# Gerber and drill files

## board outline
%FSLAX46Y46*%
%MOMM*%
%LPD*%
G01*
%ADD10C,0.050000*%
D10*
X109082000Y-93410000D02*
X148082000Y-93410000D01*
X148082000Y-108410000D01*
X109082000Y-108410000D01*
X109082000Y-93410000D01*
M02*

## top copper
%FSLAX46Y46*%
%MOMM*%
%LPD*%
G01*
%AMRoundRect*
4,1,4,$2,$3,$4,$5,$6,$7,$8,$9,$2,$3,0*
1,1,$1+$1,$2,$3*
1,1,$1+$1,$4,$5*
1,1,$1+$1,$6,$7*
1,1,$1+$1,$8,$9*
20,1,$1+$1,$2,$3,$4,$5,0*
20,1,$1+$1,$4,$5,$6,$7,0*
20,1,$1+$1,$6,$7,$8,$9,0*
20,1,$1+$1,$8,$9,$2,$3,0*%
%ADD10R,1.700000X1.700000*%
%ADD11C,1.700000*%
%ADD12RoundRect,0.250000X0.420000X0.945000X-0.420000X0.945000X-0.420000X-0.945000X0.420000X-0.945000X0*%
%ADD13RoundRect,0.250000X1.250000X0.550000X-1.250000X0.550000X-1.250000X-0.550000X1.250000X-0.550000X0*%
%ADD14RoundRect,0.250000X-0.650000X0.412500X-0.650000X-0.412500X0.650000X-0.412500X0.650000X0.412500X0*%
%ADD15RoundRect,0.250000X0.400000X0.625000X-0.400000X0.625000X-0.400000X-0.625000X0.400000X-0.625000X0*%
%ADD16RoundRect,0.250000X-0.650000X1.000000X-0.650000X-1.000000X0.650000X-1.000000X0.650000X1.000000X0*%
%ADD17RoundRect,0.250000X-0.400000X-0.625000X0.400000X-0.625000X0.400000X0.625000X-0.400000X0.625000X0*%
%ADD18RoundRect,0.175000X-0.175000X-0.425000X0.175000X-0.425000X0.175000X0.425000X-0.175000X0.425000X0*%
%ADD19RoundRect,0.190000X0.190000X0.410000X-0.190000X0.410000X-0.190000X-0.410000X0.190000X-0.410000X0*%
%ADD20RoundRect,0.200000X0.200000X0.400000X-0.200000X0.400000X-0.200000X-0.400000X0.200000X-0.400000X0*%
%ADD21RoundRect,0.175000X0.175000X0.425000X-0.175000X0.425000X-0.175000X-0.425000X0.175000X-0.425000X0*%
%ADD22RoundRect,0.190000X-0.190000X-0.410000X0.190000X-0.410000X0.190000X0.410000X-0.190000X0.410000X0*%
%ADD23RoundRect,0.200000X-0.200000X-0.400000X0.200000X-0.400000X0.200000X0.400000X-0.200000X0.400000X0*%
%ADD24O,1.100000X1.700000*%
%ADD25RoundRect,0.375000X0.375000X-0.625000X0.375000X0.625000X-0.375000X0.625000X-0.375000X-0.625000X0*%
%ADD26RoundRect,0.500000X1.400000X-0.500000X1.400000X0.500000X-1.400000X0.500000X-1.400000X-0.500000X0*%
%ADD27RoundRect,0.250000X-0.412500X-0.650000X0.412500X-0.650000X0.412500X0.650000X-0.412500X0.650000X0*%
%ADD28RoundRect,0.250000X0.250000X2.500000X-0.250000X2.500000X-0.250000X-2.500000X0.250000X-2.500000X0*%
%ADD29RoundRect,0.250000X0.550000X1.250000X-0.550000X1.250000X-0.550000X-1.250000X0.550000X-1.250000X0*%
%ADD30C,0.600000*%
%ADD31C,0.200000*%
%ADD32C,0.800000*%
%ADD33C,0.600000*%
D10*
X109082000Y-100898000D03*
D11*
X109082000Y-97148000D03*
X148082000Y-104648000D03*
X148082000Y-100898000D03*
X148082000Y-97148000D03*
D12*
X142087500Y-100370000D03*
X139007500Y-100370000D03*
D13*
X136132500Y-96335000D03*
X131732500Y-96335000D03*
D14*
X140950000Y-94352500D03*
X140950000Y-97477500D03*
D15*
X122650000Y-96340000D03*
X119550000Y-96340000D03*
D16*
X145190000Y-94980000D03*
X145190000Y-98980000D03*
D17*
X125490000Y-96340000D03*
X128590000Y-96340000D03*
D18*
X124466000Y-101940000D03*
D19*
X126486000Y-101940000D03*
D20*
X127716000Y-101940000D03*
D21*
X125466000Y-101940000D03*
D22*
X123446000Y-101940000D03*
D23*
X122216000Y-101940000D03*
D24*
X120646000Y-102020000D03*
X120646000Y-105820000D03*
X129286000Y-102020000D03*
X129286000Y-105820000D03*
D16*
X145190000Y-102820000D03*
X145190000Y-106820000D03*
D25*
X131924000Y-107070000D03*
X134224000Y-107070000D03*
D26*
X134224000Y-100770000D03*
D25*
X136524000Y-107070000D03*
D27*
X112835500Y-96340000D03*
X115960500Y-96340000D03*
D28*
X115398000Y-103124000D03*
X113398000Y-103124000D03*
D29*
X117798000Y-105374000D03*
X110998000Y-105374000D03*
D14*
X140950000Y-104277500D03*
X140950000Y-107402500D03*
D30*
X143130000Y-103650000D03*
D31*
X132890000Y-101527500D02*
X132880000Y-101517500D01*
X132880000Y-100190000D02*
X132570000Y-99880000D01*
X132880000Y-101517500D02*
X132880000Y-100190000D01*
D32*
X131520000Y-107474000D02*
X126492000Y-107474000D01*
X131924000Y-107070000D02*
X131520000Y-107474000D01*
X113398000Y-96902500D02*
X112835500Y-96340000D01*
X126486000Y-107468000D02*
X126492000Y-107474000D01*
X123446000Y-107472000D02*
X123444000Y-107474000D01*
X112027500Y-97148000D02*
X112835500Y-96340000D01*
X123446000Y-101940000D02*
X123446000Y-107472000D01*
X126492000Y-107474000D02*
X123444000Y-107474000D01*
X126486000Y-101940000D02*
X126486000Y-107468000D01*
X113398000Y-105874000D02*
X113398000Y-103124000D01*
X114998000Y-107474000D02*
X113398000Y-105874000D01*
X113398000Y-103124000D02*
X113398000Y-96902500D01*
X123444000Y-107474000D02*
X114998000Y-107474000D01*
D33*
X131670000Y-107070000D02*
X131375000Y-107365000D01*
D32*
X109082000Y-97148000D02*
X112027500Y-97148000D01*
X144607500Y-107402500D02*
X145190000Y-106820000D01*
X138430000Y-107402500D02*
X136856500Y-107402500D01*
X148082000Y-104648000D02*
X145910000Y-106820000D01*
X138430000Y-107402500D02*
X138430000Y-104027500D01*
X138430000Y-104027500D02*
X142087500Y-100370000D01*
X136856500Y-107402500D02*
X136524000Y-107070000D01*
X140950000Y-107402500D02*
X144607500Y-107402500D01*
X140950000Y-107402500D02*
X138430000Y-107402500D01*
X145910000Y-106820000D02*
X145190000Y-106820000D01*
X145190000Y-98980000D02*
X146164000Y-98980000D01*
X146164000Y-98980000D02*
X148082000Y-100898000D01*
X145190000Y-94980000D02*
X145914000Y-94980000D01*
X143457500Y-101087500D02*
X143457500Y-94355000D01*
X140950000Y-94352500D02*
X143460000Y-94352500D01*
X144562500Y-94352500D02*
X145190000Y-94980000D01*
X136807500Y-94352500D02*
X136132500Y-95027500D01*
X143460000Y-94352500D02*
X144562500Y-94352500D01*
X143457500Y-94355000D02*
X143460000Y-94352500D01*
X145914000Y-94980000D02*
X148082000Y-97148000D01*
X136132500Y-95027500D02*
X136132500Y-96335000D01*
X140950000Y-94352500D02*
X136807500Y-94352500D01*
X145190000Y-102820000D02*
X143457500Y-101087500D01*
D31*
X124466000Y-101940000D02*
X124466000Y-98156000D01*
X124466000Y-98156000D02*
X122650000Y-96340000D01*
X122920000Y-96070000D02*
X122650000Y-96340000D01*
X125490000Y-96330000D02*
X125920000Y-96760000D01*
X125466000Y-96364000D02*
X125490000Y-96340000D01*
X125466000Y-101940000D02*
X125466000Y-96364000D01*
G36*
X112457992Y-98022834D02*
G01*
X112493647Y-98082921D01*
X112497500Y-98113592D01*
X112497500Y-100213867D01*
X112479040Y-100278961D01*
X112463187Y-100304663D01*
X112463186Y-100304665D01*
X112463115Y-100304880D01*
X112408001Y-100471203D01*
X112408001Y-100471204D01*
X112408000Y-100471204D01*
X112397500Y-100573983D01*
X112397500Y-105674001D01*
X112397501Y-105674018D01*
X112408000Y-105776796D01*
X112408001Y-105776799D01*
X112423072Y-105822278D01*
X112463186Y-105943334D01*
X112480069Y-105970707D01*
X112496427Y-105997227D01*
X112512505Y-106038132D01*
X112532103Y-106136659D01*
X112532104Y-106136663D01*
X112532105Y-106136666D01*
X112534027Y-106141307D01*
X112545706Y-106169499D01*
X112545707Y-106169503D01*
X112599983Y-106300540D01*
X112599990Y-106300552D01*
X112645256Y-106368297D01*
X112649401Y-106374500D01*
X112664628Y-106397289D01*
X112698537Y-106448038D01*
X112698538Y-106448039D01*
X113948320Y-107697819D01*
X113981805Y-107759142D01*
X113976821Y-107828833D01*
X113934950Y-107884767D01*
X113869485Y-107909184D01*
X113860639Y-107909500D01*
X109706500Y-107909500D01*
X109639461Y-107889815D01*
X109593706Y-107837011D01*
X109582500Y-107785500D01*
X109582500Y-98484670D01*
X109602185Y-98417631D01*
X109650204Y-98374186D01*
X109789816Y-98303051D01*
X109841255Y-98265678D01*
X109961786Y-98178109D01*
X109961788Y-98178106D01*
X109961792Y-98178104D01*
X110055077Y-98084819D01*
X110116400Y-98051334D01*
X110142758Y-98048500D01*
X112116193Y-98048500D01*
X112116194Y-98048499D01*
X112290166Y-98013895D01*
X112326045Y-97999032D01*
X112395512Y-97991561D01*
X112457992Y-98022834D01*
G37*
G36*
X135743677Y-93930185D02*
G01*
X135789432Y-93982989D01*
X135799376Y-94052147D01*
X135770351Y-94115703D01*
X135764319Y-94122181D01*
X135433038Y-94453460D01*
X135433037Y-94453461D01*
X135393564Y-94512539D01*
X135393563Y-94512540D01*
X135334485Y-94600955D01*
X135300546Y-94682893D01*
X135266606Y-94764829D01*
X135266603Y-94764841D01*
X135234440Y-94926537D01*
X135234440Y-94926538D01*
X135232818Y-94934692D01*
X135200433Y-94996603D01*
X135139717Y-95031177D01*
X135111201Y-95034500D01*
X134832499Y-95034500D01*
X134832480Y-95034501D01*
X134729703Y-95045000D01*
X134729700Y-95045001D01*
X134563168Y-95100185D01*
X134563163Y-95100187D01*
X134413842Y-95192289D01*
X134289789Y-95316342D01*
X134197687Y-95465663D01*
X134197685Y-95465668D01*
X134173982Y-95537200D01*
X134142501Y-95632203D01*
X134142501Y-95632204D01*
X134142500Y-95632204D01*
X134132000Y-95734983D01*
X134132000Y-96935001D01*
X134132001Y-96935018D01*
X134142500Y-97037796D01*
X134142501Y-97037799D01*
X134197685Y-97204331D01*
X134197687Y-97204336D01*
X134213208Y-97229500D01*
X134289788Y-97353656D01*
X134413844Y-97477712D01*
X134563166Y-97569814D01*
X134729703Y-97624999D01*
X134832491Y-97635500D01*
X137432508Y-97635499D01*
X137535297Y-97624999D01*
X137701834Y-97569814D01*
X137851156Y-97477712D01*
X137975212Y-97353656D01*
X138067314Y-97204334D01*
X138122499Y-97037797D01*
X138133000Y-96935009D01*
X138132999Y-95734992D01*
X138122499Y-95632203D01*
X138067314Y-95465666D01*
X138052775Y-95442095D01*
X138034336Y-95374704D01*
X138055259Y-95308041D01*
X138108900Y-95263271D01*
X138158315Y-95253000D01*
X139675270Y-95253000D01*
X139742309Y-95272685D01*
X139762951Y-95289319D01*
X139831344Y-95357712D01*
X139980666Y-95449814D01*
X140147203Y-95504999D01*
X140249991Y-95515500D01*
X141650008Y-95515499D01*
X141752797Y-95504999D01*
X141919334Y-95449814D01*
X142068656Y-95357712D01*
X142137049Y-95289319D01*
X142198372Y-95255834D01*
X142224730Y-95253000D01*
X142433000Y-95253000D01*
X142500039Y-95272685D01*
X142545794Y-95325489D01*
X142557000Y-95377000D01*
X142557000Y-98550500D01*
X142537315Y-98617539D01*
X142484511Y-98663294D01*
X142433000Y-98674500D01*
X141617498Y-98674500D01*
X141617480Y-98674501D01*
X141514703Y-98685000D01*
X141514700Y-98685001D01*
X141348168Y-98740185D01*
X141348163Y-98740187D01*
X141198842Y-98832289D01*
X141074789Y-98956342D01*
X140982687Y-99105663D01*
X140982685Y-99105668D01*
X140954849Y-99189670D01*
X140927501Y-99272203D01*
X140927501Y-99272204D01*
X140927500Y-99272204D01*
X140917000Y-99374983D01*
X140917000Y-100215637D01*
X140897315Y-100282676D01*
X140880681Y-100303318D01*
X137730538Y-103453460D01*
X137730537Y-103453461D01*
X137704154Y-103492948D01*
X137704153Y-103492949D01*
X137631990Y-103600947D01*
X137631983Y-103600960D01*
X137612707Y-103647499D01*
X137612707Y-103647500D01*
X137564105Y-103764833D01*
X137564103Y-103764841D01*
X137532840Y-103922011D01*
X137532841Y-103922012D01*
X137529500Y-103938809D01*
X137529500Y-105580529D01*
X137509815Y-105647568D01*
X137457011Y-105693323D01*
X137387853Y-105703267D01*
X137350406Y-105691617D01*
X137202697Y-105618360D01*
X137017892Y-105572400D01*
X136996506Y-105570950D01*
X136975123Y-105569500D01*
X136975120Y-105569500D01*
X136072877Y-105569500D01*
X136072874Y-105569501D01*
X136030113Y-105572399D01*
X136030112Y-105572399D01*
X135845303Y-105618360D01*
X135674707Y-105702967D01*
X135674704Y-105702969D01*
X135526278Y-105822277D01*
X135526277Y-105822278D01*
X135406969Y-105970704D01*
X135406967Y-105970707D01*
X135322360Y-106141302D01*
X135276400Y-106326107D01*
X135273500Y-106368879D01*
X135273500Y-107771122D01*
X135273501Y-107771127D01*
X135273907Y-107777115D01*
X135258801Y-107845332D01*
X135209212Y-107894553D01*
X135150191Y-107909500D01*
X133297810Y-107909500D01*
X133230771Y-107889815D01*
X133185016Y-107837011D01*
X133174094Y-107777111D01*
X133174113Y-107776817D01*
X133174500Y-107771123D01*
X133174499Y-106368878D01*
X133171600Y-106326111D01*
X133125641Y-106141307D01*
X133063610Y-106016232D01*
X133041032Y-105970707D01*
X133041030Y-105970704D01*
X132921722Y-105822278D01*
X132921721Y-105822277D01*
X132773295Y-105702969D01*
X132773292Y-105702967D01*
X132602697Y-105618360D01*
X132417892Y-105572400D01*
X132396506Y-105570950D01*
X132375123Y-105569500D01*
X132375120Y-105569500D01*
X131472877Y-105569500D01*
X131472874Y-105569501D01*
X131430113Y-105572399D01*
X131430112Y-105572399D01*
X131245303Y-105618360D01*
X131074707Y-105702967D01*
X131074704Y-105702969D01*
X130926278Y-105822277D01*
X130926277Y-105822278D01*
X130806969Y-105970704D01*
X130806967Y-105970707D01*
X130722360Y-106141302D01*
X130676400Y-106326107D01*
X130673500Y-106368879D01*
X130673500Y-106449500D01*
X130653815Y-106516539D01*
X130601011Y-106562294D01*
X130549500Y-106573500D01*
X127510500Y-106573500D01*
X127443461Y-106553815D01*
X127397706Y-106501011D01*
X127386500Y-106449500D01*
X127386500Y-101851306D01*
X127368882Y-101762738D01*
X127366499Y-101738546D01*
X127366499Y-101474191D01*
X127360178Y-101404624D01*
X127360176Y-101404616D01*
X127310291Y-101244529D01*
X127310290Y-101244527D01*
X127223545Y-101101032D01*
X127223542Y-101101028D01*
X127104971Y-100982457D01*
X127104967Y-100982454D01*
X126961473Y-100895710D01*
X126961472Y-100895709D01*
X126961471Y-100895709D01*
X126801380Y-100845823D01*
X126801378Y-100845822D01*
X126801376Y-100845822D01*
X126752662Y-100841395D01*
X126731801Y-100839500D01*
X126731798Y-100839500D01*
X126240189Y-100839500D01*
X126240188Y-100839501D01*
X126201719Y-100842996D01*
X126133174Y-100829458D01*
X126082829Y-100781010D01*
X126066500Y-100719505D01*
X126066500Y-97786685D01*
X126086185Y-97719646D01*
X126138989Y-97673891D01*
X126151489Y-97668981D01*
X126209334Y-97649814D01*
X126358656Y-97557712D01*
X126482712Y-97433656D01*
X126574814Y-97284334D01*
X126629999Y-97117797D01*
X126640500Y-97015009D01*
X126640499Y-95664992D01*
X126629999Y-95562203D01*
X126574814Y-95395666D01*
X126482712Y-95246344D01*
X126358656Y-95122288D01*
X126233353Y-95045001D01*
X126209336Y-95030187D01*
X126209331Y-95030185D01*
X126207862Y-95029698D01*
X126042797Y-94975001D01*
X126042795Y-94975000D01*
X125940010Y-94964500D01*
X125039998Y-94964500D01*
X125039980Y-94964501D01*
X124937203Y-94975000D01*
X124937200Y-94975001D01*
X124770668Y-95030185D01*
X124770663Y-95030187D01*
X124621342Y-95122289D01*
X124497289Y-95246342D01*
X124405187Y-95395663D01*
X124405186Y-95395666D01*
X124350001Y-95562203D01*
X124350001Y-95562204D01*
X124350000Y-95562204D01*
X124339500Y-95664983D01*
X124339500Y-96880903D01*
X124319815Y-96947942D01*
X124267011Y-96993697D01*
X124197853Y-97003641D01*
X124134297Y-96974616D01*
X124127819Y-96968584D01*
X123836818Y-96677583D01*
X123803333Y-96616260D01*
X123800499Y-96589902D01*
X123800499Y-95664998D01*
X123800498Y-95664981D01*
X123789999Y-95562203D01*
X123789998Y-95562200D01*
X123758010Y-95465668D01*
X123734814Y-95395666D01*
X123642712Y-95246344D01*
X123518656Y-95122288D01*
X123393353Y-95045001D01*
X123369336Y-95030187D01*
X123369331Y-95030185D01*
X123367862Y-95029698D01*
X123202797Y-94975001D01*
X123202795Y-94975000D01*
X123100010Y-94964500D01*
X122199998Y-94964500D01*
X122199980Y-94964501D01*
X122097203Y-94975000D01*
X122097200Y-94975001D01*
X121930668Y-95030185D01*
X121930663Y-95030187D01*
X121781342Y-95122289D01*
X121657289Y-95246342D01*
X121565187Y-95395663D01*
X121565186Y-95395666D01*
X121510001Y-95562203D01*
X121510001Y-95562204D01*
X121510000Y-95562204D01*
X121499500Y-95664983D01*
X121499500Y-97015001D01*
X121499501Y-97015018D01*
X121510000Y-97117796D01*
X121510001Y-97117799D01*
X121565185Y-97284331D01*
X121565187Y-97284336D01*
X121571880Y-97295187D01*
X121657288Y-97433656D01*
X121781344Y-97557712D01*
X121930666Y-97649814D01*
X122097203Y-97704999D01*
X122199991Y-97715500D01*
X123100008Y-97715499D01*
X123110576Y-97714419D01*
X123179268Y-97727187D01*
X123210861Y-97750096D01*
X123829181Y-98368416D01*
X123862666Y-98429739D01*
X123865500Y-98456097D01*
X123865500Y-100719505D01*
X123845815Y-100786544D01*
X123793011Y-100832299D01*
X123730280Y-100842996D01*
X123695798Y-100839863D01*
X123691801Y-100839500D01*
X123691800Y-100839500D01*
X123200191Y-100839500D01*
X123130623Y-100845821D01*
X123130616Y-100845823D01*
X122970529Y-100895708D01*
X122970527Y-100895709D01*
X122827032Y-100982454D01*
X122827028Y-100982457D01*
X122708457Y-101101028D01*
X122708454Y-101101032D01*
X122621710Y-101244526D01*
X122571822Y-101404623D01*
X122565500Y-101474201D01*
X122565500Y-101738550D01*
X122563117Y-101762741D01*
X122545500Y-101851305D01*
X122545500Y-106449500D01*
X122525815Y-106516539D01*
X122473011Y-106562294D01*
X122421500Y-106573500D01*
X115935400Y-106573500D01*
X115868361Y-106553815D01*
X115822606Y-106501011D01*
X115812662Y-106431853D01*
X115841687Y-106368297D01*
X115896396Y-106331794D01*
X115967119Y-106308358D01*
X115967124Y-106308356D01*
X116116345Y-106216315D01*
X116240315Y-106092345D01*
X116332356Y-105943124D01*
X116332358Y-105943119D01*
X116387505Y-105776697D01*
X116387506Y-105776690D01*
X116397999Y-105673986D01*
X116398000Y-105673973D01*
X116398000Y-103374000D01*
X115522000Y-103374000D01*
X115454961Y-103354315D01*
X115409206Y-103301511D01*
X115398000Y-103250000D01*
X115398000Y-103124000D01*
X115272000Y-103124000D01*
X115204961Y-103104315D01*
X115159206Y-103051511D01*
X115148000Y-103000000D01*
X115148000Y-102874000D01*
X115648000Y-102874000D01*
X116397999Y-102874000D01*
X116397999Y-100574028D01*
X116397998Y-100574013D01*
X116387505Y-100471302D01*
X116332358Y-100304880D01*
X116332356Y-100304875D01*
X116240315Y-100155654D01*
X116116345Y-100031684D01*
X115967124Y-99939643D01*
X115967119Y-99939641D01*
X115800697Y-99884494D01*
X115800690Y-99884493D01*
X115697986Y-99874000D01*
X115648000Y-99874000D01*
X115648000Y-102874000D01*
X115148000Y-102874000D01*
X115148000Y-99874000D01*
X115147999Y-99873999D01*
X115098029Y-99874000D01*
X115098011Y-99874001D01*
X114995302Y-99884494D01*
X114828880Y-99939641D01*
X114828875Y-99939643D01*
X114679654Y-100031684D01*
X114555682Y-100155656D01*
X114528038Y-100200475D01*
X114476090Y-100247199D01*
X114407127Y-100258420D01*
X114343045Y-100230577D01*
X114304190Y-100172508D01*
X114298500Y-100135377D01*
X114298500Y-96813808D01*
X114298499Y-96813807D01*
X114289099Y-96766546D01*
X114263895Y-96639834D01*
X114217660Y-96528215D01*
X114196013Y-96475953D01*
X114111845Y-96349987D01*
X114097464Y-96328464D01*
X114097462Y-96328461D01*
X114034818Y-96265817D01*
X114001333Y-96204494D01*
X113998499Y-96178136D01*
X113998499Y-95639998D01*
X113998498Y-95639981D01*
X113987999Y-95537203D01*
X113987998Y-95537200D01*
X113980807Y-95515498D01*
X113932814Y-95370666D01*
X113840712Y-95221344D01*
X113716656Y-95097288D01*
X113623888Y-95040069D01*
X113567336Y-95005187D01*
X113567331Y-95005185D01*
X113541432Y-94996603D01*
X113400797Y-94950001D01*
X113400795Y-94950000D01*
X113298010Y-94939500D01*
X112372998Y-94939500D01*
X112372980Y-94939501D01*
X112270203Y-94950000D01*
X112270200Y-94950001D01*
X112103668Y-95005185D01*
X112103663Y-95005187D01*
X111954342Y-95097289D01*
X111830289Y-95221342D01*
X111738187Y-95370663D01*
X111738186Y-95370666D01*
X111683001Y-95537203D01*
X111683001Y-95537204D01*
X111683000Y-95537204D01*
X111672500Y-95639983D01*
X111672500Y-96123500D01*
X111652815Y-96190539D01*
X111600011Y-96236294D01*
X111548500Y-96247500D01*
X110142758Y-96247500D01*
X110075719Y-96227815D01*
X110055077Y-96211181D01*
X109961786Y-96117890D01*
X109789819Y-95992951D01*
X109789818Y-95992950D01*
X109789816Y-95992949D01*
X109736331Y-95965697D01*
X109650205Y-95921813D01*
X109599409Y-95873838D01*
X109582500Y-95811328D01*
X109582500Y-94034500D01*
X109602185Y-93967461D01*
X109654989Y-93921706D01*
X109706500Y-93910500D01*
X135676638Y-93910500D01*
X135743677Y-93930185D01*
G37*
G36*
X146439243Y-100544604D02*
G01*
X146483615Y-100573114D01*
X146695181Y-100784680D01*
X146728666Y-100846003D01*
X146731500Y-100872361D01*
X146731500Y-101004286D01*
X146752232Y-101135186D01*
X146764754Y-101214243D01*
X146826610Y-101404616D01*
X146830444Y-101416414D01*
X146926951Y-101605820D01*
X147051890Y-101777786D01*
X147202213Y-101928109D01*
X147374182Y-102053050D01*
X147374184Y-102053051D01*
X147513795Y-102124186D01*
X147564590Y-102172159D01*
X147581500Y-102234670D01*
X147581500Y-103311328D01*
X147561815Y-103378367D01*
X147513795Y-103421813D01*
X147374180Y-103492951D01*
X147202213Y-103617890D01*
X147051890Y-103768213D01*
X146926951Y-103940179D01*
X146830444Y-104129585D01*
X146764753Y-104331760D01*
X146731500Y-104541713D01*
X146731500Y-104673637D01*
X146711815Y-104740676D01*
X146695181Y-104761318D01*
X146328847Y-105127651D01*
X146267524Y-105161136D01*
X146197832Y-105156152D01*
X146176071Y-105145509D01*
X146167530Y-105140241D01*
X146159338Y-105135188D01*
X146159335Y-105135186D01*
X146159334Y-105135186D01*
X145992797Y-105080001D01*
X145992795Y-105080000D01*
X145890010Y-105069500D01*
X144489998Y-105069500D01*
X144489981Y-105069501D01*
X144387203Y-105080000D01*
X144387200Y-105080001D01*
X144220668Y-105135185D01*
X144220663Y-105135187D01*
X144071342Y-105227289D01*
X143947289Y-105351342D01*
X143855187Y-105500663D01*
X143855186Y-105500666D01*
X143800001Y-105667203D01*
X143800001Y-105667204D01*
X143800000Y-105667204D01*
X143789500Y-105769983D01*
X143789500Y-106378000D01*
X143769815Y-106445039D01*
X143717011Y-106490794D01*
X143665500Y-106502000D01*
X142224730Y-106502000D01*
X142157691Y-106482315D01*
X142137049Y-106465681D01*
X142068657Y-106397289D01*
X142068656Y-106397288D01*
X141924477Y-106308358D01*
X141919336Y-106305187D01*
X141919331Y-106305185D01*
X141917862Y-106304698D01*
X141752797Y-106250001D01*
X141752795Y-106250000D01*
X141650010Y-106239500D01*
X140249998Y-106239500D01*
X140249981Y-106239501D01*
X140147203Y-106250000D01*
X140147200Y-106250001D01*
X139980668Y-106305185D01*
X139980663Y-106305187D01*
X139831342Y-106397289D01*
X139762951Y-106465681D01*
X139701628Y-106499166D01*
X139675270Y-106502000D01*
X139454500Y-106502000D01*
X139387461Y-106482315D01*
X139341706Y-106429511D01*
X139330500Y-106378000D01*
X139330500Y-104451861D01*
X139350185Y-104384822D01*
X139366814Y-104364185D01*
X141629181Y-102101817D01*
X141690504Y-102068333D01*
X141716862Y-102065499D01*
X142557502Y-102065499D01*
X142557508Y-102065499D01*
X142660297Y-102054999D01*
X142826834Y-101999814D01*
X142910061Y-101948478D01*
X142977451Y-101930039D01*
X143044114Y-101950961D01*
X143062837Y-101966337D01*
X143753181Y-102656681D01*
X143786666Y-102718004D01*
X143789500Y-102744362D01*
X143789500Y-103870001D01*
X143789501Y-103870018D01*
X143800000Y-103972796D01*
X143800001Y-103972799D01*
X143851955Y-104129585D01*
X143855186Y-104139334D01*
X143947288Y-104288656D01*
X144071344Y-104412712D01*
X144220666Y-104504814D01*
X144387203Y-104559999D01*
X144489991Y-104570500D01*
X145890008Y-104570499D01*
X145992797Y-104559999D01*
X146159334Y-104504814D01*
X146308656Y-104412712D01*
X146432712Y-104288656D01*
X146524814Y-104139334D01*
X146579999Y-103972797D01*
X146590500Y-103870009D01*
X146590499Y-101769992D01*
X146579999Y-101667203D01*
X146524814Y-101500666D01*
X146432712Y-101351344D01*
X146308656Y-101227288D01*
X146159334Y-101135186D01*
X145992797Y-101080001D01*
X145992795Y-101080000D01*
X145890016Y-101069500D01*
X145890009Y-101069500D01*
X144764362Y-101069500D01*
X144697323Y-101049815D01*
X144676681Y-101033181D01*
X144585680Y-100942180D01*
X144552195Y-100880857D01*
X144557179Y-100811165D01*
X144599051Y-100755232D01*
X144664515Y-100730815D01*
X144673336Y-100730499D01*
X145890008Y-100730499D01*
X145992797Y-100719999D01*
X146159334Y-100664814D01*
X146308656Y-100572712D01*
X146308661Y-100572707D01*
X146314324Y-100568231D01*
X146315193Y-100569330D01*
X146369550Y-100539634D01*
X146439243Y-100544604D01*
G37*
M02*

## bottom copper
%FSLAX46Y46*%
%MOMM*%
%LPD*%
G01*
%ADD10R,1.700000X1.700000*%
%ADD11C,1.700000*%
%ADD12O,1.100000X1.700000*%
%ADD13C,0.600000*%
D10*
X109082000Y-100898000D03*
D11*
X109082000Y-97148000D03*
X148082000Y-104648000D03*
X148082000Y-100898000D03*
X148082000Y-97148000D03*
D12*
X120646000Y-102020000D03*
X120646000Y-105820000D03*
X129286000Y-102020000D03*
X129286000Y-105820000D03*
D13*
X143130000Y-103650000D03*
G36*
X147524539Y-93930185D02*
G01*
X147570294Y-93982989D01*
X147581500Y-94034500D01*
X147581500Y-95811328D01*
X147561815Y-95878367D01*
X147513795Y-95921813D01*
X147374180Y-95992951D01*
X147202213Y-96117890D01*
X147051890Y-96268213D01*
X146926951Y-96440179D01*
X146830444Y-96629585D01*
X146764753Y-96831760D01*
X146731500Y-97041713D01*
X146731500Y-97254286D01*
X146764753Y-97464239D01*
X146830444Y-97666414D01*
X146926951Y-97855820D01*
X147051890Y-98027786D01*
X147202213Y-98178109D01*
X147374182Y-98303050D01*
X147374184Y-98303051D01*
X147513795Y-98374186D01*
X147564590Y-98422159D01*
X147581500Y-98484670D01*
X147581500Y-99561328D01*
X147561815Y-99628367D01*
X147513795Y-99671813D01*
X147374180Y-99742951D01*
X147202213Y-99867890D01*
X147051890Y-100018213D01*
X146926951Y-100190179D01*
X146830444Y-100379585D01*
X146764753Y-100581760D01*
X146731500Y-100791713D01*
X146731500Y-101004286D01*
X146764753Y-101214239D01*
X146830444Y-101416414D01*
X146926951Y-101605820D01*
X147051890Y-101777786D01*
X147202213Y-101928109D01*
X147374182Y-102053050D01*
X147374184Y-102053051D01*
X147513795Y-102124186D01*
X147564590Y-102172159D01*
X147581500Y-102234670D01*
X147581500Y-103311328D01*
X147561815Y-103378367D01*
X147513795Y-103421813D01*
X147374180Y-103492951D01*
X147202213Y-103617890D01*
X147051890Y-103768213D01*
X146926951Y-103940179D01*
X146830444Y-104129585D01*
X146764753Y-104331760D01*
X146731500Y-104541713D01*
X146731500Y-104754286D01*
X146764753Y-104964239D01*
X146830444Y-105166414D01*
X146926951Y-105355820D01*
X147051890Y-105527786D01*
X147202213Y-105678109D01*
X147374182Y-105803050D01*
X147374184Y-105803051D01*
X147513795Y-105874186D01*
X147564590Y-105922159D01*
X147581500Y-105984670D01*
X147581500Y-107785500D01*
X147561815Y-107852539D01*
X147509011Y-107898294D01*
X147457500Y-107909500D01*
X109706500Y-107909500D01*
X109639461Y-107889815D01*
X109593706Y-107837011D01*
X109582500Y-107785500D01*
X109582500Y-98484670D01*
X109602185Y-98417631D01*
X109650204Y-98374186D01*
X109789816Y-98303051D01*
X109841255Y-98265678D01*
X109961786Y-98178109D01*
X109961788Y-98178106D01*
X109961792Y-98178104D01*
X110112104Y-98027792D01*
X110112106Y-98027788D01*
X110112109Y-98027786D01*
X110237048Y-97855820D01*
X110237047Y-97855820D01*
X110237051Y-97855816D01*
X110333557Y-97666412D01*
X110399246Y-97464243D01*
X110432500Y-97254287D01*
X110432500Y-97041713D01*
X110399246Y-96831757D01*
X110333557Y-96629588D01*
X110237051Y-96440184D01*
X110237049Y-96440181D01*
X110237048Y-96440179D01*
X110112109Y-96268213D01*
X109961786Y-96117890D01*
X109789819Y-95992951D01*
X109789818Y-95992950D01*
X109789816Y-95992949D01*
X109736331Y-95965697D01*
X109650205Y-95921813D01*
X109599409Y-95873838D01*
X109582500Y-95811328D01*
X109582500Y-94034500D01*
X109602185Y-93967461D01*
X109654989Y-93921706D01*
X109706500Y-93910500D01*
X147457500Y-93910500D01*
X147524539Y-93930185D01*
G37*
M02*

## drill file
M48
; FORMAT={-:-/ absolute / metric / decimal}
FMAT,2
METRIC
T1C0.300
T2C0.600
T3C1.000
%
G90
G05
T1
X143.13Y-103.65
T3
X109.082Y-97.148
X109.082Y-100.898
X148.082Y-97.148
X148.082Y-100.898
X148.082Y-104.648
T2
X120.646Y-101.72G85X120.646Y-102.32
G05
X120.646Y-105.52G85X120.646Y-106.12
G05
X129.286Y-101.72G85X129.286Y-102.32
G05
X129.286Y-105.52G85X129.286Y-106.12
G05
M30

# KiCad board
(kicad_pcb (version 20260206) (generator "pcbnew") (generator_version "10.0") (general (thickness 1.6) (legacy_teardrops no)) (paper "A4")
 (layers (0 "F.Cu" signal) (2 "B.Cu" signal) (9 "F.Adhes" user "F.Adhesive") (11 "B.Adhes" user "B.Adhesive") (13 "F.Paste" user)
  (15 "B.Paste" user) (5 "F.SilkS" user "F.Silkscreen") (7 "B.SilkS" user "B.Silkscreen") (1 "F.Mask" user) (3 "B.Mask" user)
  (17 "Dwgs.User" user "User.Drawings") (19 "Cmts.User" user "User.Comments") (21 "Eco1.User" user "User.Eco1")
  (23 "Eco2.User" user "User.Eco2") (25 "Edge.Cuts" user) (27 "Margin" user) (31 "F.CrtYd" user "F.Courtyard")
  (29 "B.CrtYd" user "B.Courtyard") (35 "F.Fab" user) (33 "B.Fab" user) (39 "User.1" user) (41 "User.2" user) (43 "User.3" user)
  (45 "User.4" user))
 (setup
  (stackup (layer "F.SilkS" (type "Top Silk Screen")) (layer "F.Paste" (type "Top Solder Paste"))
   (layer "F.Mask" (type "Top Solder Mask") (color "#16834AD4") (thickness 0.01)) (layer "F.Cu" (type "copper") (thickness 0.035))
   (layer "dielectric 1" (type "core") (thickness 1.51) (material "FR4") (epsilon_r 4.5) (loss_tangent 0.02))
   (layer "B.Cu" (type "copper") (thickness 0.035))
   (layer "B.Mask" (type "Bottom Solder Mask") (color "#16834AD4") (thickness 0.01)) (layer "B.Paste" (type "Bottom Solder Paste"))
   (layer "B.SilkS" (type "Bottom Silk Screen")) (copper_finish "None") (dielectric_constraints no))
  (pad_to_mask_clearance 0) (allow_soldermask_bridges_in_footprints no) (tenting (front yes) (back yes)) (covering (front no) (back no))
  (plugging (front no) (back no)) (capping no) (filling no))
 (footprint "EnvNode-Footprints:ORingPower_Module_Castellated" (layer "F.Cu") (at 128.582 100.898)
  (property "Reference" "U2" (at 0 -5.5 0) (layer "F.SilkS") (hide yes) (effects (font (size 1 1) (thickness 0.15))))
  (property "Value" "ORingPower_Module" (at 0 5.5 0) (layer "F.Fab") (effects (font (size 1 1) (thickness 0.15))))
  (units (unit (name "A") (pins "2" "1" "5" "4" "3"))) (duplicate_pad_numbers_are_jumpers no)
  (pad "1" thru_hole rect (at -19.5 0) (size 1.7 1.7) (drill 1) (layers "*.Cu" "*.Mask") (remove_unused_layers no) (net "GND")
   (zone_connect 2))
  (pad "2" thru_hole circle (at -19.5 -3.75) (size 1.7 1.7) (drill 1) (layers "*.Cu" "*.Mask") (remove_unused_layers no) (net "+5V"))
  (pad "3" thru_hole circle (at 19.5 3.75) (size 1.7 1.7) (drill 1) (layers "*.Cu" "*.Mask") (remove_unused_layers no) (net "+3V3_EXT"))
  (pad "4" thru_hole circle (at 19.5 0) (size 1.7 1.7) (drill 1) (layers "*.Cu" "*.Mask") (remove_unused_layers no) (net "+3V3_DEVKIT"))
  (pad "5" thru_hole circle (at 19.5 -3.75) (size 1.7 1.7) (drill 1) (layers "*.Cu" "*.Mask") (remove_unused_layers no) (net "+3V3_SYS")))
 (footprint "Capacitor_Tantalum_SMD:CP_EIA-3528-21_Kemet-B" (layer "F.Cu") (at 140.5475 100.37 180)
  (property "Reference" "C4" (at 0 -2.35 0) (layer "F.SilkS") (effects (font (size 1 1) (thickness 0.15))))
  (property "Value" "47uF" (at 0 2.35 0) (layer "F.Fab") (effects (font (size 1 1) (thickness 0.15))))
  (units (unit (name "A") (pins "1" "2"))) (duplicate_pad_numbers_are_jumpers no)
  (pad "1" smd roundrect (at -1.54 0 180) (size 1.34 2.39) (layers "F.Cu" "F.Mask" "F.Paste") (roundrect_rratio 0.186567) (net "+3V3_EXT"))
  (pad "2" smd roundrect (at 1.54 0 180) (size 1.34 2.39) (layers "F.Cu" "F.Mask" "F.Paste") (roundrect_rratio 0.186567) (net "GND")
   (zone_connect 2)))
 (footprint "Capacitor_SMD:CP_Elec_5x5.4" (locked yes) (layer "F.Cu") (at 133.9325 96.335 180)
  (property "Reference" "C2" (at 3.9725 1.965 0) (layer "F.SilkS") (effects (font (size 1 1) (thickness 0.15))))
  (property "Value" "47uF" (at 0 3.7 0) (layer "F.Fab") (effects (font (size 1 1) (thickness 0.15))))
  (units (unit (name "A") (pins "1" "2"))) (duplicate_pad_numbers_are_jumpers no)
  (pad "1" smd roundrect (at -2.2 0 180) (size 3 1.6) (layers "F.Cu" "F.Mask" "F.Paste") (roundrect_rratio 0.15625) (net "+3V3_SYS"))
  (pad "2" smd roundrect (at 2.2 0 180) (size 3 1.6) (layers "F.Cu" "F.Mask" "F.Paste") (roundrect_rratio 0.15625) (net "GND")
   (zone_connect 2)))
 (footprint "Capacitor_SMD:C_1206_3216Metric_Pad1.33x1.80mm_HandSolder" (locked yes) (layer "F.Cu") (at 140.95 95.915 -90)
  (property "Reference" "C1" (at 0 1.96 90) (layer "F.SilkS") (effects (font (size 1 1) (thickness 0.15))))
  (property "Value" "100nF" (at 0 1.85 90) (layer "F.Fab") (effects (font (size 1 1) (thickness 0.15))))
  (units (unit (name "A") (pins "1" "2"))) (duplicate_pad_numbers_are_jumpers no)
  (pad "1" smd roundrect (at -1.5625 0 270) (size 1.325 1.8) (layers "F.Cu" "F.Mask" "F.Paste") (roundrect_rratio 0.188679) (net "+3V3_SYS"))
  (pad "2" smd roundrect (at 1.5625 0 270) (size 1.325 1.8) (layers "F.Cu" "F.Mask" "F.Paste") (roundrect_rratio 0.188679) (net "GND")
   (zone_connect 2)))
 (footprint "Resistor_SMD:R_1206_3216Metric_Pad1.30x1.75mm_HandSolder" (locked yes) (layer "F.Cu") (at 121.1 96.34 180)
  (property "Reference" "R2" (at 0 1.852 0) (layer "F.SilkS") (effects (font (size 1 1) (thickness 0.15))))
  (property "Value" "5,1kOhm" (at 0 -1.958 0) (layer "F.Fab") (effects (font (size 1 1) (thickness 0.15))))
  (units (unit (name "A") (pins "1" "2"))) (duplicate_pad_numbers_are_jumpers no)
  (pad "1" smd roundrect (at -1.55 0 180) (size 1.3 1.75) (layers "F.Cu" "F.Mask" "F.Paste") (roundrect_rratio 0.192308)
   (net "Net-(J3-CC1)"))
  (pad "2" smd roundrect (at 1.55 0 180) (size 1.3 1.75) (layers "F.Cu" "F.Mask" "F.Paste") (roundrect_rratio 0.192308) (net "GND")
   (zone_connect 2)))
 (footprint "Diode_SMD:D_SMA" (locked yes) (layer "F.Cu") (at 145.19 96.98 -90)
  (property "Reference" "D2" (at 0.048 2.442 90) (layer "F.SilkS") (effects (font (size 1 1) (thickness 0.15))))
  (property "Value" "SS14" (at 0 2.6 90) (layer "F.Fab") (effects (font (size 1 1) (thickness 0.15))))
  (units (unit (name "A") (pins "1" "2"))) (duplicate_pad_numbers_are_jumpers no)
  (pad "1" smd roundrect (at -2 0 270) (size 2.5 1.8) (layers "F.Cu" "F.Mask" "F.Paste") (roundrect_rratio 0.1388888889) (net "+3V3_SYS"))
  (pad "2" smd roundrect (at 2 0 270) (size 2.5 1.8) (layers "F.Cu" "F.Mask" "F.Paste") (roundrect_rratio 0.1388888889) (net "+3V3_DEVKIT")))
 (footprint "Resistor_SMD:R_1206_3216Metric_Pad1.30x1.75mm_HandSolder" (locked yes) (layer "F.Cu") (at 127.04 96.34)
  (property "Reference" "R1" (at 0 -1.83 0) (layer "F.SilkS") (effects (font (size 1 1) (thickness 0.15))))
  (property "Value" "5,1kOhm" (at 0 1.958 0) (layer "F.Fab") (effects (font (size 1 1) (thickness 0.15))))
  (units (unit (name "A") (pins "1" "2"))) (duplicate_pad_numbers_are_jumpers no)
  (pad "1" smd roundrect (at -1.55 0) (size 1.3 1.75) (layers "F.Cu" "F.Mask" "F.Paste") (roundrect_rratio 0.192308) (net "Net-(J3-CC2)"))
  (pad "2" smd roundrect (at 1.55 0) (size 1.3 1.75) (layers "F.Cu" "F.Mask" "F.Paste") (roundrect_rratio 0.192308) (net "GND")
   (zone_connect 2)))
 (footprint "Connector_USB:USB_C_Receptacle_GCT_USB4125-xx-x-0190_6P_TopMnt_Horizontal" (layer "F.Cu") (at 124.966 105.02)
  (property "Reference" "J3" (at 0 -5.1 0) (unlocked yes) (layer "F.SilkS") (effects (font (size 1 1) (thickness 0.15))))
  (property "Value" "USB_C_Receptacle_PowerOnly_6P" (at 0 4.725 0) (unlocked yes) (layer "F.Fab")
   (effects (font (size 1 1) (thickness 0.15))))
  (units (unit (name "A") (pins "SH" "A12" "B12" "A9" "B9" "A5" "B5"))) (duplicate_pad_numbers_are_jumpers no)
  (pad "A5" smd roundrect (at -0.5 -3.08) (size 0.7 1.2) (layers "F.Cu" "F.Mask" "F.Paste") (roundrect_rratio 0.25) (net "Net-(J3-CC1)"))
  (pad "A9" smd roundrect (at 1.52 -3.08 180) (size 0.76 1.2) (layers "F.Cu" "F.Mask" "F.Paste") (roundrect_rratio 0.25) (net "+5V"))
  (pad "A12" smd roundrect (at 2.75 -3.08 180) (size 0.8 1.2) (layers "F.Cu" "F.Mask" "F.Paste") (roundrect_rratio 0.25) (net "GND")
   (zone_connect 2))
  (pad "B5" smd roundrect (at 0.5 -3.08 180) (size 0.7 1.2) (layers "F.Cu" "F.Mask" "F.Paste") (roundrect_rratio 0.25) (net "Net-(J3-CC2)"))
  (pad "B9" smd roundrect (at -1.52 -3.08) (size 0.76 1.2) (layers "F.Cu" "F.Mask" "F.Paste") (roundrect_rratio 0.25) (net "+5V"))
  (pad "B12" smd roundrect (at -2.75 -3.08) (size 0.8 1.2) (layers "F.Cu" "F.Mask" "F.Paste") (roundrect_rratio 0.25) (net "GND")
   (zone_connect 2))
  (pad "SH" thru_hole oval (at -4.32 -3) (size 1.1 1.7) (drill oval 0.6 1.2) (layers "*.Cu" "*.Mask" "F.Paste") (remove_unused_layers no)
   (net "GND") (zone_connect 2))
  (pad "SH" thru_hole oval (at -4.32 0.8) (size 1.1 1.7) (drill oval 0.6 1.2) (layers "*.Cu" "*.Mask" "F.Paste") (remove_unused_layers no)
   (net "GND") (zone_connect 2))
  (pad "SH" thru_hole oval (at 4.32 -3) (size 1.1 1.7) (drill oval 0.6 1.2) (layers "*.Cu" "*.Mask" "F.Paste") (remove_unused_layers no)
   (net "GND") (zone_connect 2))
  (pad "SH" thru_hole oval (at 4.32 0.8) (size 1.1 1.7) (drill oval 0.6 1.2) (layers "*.Cu" "*.Mask" "F.Paste") (remove_unused_layers no)
   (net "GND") (zone_connect 2)))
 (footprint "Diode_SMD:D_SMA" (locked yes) (layer "F.Cu") (at 145.19 104.82 -90)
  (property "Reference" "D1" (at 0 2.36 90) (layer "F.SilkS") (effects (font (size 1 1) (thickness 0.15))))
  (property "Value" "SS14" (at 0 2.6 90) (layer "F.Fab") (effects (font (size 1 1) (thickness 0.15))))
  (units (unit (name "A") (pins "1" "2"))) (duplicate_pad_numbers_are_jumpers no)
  (pad "1" smd roundrect (at -2 0 270) (size 2.5 1.8) (layers "F.Cu" "F.Mask" "F.Paste") (roundrect_rratio 0.1388888889) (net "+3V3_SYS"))
  (pad "2" smd roundrect (at 2 0 270) (size 2.5 1.8) (layers "F.Cu" "F.Mask" "F.Paste") (roundrect_rratio 0.1388888889) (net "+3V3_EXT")))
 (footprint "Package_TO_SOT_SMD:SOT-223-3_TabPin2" (layer "F.Cu") (at 134.224 103.92 90)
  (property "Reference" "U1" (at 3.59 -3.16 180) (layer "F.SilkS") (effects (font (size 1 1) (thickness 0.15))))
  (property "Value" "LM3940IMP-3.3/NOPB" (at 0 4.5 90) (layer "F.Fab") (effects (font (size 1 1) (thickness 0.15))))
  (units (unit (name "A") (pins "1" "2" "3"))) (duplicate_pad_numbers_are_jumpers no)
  (pad "1" smd roundrect (at -3.15 -2.3 90) (size 2 1.5) (layers "F.Cu" "F.Mask" "F.Paste") (roundrect_rratio 0.25) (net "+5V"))
  (pad "2" smd roundrect (at -3.15 0 90) (size 2 1.5) (layers "F.Cu" "F.Mask" "F.Paste") (roundrect_rratio 0.25) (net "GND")
   (zone_connect 2))
  (pad "2" smd roundrect (at 3.15 0 90) (size 2 3.8) (layers "F.Cu" "F.Mask" "F.Paste") (roundrect_rratio 0.25) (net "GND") (zone_connect 2))
  (pad "3" smd roundrect (at -3.15 2.3 90) (size 2 1.5) (layers "F.Cu" "F.Mask" "F.Paste") (roundrect_rratio 0.25) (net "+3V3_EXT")))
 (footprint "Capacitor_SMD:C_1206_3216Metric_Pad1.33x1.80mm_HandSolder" (layer "F.Cu") (at 114.398 96.34)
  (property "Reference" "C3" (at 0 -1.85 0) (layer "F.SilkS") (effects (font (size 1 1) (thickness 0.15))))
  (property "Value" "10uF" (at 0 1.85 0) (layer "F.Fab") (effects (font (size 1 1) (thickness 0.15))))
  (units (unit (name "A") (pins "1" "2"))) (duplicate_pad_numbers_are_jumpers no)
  (pad "1" smd roundrect (at -1.5625 0) (size 1.325 1.8) (layers "F.Cu" "F.Mask" "F.Paste") (roundrect_rratio 0.188679) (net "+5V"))
  (pad "2" smd roundrect (at 1.5625 0) (size 1.325 1.8) (layers "F.Cu" "F.Mask" "F.Paste") (roundrect_rratio 0.188679) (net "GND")
   (zone_connect 2)))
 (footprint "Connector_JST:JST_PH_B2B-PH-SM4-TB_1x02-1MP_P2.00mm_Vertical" (layer "F.Cu") (at 114.398 103.624 180)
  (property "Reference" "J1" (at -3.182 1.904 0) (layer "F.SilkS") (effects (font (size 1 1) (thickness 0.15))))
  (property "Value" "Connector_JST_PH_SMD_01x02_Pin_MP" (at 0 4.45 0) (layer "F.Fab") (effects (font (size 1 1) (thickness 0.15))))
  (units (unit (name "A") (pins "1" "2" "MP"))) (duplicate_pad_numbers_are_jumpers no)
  (pad "1" smd roundrect (at -1 0.5 180) (size 1 5.5) (layers "F.Cu" "F.Mask" "F.Paste") (roundrect_rratio 0.25) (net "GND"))
  (pad "2" smd roundrect (at 1 0.5 180) (size 1 5.5) (layers "F.Cu" "F.Mask" "F.Paste") (roundrect_rratio 0.25) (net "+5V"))
  (pad "MP" smd roundrect (at -3.4 -1.75 180) (size 1.6 3) (layers "F.Cu" "F.Mask" "F.Paste") (roundrect_rratio 0.15625) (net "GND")
   (zone_connect 2))
  (pad "MP" smd roundrect (at 3.4 -1.75 180) (size 1.6 3) (layers "F.Cu" "F.Mask" "F.Paste") (roundrect_rratio 0.15625) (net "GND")
   (zone_connect 2)))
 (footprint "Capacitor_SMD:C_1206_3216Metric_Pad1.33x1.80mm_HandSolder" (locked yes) (layer "F.Cu") (at 140.95 105.84 -90)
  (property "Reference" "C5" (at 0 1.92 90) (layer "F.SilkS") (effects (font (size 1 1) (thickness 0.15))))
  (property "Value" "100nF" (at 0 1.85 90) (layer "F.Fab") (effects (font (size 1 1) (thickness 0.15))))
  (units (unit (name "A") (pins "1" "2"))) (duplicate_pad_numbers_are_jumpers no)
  (pad "1" smd roundrect (at -1.5625 0 270) (size 1.325 1.8) (layers "F.Cu" "F.Mask" "F.Paste") (roundrect_rratio 0.188679) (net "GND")
   (zone_connect 2))
  (pad "2" smd roundrect (at 1.5625 0 270) (size 1.325 1.8) (layers "F.Cu" "F.Mask" "F.Paste") (roundrect_rratio 0.188679) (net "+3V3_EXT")))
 (gr_rect (start 109.082 93.41) (end 148.082 108.41) (stroke (width 0.05) (type solid)) (fill no) (layer "Edge.Cuts"))
 (segment (start 132.89 101.5275) (end 132.88 101.5175) (width 0.2) (layer "F.Cu") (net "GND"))
 (segment (start 132.88 100.19) (end 132.57 99.88) (width 0.2) (layer "F.Cu") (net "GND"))
 (segment (start 132.88 101.5175) (end 132.88 100.19) (width 0.2) (layer "F.Cu") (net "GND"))
 (via (at 143.13 103.65) (size 0.6) (drill 0.3) (layers "F.Cu" "B.Cu") (free yes) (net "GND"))
 (segment (start 131.52 107.474) (end 126.492 107.474) (width 0.8) (layer "F.Cu") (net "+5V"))
 (segment (start 131.924 107.07) (end 131.52 107.474) (width 0.8) (layer "F.Cu") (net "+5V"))
 (segment (start 113.398 96.9025) (end 112.8355 96.34) (width 0.8) (layer "F.Cu") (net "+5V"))
 (segment (start 126.486 107.468) (end 126.492 107.474) (width 0.8) (layer "F.Cu") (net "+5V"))
 (segment (start 123.446 107.472) (end 123.444 107.474) (width 0.8) (layer "F.Cu") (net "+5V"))
 (segment (start 112.0275 97.148) (end 112.8355 96.34) (width 0.8) (layer "F.Cu") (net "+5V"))
 (segment (start 123.446 101.94) (end 123.446 107.472) (width 0.8) (layer "F.Cu") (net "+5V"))
 (segment (start 126.492 107.474) (end 123.444 107.474) (width 0.8) (layer "F.Cu") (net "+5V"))
 (segment (start 126.486 101.94) (end 126.486 107.468) (width 0.8) (layer "F.Cu") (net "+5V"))
 (segment (start 113.398 105.874) (end 113.398 103.124) (width 0.8) (layer "F.Cu") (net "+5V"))
 (segment (start 114.998 107.474) (end 113.398 105.874) (width 0.8) (layer "F.Cu") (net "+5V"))
 (segment (start 113.398 103.124) (end 113.398 96.9025) (width 0.8) (layer "F.Cu") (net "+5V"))
 (segment (start 123.444 107.474) (end 114.998 107.474) (width 0.8) (layer "F.Cu") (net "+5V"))
 (segment (start 131.67 107.07) (end 131.375 107.365) (width 0.6) (layer "F.Cu") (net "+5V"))
 (segment (start 109.082 97.148) (end 112.0275 97.148) (width 0.8) (layer "F.Cu") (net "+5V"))
 (segment (start 144.6075 107.4025) (end 145.19 106.82) (width 0.8) (layer "F.Cu") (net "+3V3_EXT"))
 (segment (start 138.43 107.4025) (end 136.8565 107.4025) (width 0.8) (layer "F.Cu") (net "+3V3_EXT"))
 (segment (start 148.082 104.648) (end 145.91 106.82) (width 0.8) (layer "F.Cu") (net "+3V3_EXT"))
 (segment (start 138.43 107.4025) (end 138.43 104.0275) (width 0.8) (layer "F.Cu") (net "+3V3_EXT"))
 (segment (start 138.43 104.0275) (end 142.0875 100.37) (width 0.8) (layer "F.Cu") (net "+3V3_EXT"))
 (segment (start 136.8565 107.4025) (end 136.524 107.07) (width 0.8) (layer "F.Cu") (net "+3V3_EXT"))
 (segment (start 140.95 107.4025) (end 144.6075 107.4025) (width 0.8) (layer "F.Cu") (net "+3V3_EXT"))
 (segment (start 140.95 107.4025) (end 138.43 107.4025) (width 0.8) (layer "F.Cu") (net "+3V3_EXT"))
 (segment (start 145.91 106.82) (end 145.19 106.82) (width 0.8) (layer "F.Cu") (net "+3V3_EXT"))
 (segment (start 145.19 98.98) (end 146.164 98.98) (width 0.8) (layer "F.Cu") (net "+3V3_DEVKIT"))
 (segment (start 146.164 98.98) (end 148.082 100.898) (width 0.8) (layer "F.Cu") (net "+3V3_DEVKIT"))
 (segment (start 145.19 94.98) (end 145.914 94.98) (width 0.8) (layer "F.Cu") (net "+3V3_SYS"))
 (segment (start 143.4575 101.0875) (end 143.4575 94.355) (width 0.8) (layer "F.Cu") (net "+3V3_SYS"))
 (segment (start 140.95 94.3525) (end 143.46 94.3525) (width 0.8) (layer "F.Cu") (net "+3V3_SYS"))
 (segment (start 144.5625 94.3525) (end 145.19 94.98) (width 0.8) (layer "F.Cu") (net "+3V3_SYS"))
 (segment (start 136.8075 94.3525) (end 136.1325 95.0275) (width 0.8) (layer "F.Cu") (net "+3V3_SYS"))
 (segment (start 143.46 94.3525) (end 144.5625 94.3525) (width 0.8) (layer "F.Cu") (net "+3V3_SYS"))
 (segment (start 143.4575 94.355) (end 143.46 94.3525) (width 0.8) (layer "F.Cu") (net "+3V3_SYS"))
 (segment (start 145.914 94.98) (end 148.082 97.148) (width 0.8) (layer "F.Cu") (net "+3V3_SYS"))
 (segment (start 136.1325 95.0275) (end 136.1325 96.335) (width 0.8) (layer "F.Cu") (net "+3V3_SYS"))
 (segment (start 140.95 94.3525) (end 136.8075 94.3525) (width 0.8) (layer "F.Cu") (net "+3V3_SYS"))
 (segment (start 145.19 102.82) (end 143.4575 101.0875) (width 0.8) (layer "F.Cu") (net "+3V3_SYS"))
 (segment (start 124.466 101.94) (end 124.466 98.156) (width 0.2) (layer "F.Cu") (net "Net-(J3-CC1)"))
 (segment (start 124.466 98.156) (end 122.65 96.34) (width 0.2) (layer "F.Cu") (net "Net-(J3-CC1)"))
 (segment (start 122.92 96.07) (end 122.65 96.34) (width 0.2) (layer "F.Cu") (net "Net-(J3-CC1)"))
 (segment (start 125.49 96.33) (end 125.92 96.76) (width 0.2) (layer "F.Cu") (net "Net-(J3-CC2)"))
 (segment (start 125.466 96.364) (end 125.49 96.34) (width 0.2) (layer "F.Cu") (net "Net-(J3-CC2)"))
 (segment (start 125.466 101.94) (end 125.466 96.364) (width 0.2) (layer "F.Cu") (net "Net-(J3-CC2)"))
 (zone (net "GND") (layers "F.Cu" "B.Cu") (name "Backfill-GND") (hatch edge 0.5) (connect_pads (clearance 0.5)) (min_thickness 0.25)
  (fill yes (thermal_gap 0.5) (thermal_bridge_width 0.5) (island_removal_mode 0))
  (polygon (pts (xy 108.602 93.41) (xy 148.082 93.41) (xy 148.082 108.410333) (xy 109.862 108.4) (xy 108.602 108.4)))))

